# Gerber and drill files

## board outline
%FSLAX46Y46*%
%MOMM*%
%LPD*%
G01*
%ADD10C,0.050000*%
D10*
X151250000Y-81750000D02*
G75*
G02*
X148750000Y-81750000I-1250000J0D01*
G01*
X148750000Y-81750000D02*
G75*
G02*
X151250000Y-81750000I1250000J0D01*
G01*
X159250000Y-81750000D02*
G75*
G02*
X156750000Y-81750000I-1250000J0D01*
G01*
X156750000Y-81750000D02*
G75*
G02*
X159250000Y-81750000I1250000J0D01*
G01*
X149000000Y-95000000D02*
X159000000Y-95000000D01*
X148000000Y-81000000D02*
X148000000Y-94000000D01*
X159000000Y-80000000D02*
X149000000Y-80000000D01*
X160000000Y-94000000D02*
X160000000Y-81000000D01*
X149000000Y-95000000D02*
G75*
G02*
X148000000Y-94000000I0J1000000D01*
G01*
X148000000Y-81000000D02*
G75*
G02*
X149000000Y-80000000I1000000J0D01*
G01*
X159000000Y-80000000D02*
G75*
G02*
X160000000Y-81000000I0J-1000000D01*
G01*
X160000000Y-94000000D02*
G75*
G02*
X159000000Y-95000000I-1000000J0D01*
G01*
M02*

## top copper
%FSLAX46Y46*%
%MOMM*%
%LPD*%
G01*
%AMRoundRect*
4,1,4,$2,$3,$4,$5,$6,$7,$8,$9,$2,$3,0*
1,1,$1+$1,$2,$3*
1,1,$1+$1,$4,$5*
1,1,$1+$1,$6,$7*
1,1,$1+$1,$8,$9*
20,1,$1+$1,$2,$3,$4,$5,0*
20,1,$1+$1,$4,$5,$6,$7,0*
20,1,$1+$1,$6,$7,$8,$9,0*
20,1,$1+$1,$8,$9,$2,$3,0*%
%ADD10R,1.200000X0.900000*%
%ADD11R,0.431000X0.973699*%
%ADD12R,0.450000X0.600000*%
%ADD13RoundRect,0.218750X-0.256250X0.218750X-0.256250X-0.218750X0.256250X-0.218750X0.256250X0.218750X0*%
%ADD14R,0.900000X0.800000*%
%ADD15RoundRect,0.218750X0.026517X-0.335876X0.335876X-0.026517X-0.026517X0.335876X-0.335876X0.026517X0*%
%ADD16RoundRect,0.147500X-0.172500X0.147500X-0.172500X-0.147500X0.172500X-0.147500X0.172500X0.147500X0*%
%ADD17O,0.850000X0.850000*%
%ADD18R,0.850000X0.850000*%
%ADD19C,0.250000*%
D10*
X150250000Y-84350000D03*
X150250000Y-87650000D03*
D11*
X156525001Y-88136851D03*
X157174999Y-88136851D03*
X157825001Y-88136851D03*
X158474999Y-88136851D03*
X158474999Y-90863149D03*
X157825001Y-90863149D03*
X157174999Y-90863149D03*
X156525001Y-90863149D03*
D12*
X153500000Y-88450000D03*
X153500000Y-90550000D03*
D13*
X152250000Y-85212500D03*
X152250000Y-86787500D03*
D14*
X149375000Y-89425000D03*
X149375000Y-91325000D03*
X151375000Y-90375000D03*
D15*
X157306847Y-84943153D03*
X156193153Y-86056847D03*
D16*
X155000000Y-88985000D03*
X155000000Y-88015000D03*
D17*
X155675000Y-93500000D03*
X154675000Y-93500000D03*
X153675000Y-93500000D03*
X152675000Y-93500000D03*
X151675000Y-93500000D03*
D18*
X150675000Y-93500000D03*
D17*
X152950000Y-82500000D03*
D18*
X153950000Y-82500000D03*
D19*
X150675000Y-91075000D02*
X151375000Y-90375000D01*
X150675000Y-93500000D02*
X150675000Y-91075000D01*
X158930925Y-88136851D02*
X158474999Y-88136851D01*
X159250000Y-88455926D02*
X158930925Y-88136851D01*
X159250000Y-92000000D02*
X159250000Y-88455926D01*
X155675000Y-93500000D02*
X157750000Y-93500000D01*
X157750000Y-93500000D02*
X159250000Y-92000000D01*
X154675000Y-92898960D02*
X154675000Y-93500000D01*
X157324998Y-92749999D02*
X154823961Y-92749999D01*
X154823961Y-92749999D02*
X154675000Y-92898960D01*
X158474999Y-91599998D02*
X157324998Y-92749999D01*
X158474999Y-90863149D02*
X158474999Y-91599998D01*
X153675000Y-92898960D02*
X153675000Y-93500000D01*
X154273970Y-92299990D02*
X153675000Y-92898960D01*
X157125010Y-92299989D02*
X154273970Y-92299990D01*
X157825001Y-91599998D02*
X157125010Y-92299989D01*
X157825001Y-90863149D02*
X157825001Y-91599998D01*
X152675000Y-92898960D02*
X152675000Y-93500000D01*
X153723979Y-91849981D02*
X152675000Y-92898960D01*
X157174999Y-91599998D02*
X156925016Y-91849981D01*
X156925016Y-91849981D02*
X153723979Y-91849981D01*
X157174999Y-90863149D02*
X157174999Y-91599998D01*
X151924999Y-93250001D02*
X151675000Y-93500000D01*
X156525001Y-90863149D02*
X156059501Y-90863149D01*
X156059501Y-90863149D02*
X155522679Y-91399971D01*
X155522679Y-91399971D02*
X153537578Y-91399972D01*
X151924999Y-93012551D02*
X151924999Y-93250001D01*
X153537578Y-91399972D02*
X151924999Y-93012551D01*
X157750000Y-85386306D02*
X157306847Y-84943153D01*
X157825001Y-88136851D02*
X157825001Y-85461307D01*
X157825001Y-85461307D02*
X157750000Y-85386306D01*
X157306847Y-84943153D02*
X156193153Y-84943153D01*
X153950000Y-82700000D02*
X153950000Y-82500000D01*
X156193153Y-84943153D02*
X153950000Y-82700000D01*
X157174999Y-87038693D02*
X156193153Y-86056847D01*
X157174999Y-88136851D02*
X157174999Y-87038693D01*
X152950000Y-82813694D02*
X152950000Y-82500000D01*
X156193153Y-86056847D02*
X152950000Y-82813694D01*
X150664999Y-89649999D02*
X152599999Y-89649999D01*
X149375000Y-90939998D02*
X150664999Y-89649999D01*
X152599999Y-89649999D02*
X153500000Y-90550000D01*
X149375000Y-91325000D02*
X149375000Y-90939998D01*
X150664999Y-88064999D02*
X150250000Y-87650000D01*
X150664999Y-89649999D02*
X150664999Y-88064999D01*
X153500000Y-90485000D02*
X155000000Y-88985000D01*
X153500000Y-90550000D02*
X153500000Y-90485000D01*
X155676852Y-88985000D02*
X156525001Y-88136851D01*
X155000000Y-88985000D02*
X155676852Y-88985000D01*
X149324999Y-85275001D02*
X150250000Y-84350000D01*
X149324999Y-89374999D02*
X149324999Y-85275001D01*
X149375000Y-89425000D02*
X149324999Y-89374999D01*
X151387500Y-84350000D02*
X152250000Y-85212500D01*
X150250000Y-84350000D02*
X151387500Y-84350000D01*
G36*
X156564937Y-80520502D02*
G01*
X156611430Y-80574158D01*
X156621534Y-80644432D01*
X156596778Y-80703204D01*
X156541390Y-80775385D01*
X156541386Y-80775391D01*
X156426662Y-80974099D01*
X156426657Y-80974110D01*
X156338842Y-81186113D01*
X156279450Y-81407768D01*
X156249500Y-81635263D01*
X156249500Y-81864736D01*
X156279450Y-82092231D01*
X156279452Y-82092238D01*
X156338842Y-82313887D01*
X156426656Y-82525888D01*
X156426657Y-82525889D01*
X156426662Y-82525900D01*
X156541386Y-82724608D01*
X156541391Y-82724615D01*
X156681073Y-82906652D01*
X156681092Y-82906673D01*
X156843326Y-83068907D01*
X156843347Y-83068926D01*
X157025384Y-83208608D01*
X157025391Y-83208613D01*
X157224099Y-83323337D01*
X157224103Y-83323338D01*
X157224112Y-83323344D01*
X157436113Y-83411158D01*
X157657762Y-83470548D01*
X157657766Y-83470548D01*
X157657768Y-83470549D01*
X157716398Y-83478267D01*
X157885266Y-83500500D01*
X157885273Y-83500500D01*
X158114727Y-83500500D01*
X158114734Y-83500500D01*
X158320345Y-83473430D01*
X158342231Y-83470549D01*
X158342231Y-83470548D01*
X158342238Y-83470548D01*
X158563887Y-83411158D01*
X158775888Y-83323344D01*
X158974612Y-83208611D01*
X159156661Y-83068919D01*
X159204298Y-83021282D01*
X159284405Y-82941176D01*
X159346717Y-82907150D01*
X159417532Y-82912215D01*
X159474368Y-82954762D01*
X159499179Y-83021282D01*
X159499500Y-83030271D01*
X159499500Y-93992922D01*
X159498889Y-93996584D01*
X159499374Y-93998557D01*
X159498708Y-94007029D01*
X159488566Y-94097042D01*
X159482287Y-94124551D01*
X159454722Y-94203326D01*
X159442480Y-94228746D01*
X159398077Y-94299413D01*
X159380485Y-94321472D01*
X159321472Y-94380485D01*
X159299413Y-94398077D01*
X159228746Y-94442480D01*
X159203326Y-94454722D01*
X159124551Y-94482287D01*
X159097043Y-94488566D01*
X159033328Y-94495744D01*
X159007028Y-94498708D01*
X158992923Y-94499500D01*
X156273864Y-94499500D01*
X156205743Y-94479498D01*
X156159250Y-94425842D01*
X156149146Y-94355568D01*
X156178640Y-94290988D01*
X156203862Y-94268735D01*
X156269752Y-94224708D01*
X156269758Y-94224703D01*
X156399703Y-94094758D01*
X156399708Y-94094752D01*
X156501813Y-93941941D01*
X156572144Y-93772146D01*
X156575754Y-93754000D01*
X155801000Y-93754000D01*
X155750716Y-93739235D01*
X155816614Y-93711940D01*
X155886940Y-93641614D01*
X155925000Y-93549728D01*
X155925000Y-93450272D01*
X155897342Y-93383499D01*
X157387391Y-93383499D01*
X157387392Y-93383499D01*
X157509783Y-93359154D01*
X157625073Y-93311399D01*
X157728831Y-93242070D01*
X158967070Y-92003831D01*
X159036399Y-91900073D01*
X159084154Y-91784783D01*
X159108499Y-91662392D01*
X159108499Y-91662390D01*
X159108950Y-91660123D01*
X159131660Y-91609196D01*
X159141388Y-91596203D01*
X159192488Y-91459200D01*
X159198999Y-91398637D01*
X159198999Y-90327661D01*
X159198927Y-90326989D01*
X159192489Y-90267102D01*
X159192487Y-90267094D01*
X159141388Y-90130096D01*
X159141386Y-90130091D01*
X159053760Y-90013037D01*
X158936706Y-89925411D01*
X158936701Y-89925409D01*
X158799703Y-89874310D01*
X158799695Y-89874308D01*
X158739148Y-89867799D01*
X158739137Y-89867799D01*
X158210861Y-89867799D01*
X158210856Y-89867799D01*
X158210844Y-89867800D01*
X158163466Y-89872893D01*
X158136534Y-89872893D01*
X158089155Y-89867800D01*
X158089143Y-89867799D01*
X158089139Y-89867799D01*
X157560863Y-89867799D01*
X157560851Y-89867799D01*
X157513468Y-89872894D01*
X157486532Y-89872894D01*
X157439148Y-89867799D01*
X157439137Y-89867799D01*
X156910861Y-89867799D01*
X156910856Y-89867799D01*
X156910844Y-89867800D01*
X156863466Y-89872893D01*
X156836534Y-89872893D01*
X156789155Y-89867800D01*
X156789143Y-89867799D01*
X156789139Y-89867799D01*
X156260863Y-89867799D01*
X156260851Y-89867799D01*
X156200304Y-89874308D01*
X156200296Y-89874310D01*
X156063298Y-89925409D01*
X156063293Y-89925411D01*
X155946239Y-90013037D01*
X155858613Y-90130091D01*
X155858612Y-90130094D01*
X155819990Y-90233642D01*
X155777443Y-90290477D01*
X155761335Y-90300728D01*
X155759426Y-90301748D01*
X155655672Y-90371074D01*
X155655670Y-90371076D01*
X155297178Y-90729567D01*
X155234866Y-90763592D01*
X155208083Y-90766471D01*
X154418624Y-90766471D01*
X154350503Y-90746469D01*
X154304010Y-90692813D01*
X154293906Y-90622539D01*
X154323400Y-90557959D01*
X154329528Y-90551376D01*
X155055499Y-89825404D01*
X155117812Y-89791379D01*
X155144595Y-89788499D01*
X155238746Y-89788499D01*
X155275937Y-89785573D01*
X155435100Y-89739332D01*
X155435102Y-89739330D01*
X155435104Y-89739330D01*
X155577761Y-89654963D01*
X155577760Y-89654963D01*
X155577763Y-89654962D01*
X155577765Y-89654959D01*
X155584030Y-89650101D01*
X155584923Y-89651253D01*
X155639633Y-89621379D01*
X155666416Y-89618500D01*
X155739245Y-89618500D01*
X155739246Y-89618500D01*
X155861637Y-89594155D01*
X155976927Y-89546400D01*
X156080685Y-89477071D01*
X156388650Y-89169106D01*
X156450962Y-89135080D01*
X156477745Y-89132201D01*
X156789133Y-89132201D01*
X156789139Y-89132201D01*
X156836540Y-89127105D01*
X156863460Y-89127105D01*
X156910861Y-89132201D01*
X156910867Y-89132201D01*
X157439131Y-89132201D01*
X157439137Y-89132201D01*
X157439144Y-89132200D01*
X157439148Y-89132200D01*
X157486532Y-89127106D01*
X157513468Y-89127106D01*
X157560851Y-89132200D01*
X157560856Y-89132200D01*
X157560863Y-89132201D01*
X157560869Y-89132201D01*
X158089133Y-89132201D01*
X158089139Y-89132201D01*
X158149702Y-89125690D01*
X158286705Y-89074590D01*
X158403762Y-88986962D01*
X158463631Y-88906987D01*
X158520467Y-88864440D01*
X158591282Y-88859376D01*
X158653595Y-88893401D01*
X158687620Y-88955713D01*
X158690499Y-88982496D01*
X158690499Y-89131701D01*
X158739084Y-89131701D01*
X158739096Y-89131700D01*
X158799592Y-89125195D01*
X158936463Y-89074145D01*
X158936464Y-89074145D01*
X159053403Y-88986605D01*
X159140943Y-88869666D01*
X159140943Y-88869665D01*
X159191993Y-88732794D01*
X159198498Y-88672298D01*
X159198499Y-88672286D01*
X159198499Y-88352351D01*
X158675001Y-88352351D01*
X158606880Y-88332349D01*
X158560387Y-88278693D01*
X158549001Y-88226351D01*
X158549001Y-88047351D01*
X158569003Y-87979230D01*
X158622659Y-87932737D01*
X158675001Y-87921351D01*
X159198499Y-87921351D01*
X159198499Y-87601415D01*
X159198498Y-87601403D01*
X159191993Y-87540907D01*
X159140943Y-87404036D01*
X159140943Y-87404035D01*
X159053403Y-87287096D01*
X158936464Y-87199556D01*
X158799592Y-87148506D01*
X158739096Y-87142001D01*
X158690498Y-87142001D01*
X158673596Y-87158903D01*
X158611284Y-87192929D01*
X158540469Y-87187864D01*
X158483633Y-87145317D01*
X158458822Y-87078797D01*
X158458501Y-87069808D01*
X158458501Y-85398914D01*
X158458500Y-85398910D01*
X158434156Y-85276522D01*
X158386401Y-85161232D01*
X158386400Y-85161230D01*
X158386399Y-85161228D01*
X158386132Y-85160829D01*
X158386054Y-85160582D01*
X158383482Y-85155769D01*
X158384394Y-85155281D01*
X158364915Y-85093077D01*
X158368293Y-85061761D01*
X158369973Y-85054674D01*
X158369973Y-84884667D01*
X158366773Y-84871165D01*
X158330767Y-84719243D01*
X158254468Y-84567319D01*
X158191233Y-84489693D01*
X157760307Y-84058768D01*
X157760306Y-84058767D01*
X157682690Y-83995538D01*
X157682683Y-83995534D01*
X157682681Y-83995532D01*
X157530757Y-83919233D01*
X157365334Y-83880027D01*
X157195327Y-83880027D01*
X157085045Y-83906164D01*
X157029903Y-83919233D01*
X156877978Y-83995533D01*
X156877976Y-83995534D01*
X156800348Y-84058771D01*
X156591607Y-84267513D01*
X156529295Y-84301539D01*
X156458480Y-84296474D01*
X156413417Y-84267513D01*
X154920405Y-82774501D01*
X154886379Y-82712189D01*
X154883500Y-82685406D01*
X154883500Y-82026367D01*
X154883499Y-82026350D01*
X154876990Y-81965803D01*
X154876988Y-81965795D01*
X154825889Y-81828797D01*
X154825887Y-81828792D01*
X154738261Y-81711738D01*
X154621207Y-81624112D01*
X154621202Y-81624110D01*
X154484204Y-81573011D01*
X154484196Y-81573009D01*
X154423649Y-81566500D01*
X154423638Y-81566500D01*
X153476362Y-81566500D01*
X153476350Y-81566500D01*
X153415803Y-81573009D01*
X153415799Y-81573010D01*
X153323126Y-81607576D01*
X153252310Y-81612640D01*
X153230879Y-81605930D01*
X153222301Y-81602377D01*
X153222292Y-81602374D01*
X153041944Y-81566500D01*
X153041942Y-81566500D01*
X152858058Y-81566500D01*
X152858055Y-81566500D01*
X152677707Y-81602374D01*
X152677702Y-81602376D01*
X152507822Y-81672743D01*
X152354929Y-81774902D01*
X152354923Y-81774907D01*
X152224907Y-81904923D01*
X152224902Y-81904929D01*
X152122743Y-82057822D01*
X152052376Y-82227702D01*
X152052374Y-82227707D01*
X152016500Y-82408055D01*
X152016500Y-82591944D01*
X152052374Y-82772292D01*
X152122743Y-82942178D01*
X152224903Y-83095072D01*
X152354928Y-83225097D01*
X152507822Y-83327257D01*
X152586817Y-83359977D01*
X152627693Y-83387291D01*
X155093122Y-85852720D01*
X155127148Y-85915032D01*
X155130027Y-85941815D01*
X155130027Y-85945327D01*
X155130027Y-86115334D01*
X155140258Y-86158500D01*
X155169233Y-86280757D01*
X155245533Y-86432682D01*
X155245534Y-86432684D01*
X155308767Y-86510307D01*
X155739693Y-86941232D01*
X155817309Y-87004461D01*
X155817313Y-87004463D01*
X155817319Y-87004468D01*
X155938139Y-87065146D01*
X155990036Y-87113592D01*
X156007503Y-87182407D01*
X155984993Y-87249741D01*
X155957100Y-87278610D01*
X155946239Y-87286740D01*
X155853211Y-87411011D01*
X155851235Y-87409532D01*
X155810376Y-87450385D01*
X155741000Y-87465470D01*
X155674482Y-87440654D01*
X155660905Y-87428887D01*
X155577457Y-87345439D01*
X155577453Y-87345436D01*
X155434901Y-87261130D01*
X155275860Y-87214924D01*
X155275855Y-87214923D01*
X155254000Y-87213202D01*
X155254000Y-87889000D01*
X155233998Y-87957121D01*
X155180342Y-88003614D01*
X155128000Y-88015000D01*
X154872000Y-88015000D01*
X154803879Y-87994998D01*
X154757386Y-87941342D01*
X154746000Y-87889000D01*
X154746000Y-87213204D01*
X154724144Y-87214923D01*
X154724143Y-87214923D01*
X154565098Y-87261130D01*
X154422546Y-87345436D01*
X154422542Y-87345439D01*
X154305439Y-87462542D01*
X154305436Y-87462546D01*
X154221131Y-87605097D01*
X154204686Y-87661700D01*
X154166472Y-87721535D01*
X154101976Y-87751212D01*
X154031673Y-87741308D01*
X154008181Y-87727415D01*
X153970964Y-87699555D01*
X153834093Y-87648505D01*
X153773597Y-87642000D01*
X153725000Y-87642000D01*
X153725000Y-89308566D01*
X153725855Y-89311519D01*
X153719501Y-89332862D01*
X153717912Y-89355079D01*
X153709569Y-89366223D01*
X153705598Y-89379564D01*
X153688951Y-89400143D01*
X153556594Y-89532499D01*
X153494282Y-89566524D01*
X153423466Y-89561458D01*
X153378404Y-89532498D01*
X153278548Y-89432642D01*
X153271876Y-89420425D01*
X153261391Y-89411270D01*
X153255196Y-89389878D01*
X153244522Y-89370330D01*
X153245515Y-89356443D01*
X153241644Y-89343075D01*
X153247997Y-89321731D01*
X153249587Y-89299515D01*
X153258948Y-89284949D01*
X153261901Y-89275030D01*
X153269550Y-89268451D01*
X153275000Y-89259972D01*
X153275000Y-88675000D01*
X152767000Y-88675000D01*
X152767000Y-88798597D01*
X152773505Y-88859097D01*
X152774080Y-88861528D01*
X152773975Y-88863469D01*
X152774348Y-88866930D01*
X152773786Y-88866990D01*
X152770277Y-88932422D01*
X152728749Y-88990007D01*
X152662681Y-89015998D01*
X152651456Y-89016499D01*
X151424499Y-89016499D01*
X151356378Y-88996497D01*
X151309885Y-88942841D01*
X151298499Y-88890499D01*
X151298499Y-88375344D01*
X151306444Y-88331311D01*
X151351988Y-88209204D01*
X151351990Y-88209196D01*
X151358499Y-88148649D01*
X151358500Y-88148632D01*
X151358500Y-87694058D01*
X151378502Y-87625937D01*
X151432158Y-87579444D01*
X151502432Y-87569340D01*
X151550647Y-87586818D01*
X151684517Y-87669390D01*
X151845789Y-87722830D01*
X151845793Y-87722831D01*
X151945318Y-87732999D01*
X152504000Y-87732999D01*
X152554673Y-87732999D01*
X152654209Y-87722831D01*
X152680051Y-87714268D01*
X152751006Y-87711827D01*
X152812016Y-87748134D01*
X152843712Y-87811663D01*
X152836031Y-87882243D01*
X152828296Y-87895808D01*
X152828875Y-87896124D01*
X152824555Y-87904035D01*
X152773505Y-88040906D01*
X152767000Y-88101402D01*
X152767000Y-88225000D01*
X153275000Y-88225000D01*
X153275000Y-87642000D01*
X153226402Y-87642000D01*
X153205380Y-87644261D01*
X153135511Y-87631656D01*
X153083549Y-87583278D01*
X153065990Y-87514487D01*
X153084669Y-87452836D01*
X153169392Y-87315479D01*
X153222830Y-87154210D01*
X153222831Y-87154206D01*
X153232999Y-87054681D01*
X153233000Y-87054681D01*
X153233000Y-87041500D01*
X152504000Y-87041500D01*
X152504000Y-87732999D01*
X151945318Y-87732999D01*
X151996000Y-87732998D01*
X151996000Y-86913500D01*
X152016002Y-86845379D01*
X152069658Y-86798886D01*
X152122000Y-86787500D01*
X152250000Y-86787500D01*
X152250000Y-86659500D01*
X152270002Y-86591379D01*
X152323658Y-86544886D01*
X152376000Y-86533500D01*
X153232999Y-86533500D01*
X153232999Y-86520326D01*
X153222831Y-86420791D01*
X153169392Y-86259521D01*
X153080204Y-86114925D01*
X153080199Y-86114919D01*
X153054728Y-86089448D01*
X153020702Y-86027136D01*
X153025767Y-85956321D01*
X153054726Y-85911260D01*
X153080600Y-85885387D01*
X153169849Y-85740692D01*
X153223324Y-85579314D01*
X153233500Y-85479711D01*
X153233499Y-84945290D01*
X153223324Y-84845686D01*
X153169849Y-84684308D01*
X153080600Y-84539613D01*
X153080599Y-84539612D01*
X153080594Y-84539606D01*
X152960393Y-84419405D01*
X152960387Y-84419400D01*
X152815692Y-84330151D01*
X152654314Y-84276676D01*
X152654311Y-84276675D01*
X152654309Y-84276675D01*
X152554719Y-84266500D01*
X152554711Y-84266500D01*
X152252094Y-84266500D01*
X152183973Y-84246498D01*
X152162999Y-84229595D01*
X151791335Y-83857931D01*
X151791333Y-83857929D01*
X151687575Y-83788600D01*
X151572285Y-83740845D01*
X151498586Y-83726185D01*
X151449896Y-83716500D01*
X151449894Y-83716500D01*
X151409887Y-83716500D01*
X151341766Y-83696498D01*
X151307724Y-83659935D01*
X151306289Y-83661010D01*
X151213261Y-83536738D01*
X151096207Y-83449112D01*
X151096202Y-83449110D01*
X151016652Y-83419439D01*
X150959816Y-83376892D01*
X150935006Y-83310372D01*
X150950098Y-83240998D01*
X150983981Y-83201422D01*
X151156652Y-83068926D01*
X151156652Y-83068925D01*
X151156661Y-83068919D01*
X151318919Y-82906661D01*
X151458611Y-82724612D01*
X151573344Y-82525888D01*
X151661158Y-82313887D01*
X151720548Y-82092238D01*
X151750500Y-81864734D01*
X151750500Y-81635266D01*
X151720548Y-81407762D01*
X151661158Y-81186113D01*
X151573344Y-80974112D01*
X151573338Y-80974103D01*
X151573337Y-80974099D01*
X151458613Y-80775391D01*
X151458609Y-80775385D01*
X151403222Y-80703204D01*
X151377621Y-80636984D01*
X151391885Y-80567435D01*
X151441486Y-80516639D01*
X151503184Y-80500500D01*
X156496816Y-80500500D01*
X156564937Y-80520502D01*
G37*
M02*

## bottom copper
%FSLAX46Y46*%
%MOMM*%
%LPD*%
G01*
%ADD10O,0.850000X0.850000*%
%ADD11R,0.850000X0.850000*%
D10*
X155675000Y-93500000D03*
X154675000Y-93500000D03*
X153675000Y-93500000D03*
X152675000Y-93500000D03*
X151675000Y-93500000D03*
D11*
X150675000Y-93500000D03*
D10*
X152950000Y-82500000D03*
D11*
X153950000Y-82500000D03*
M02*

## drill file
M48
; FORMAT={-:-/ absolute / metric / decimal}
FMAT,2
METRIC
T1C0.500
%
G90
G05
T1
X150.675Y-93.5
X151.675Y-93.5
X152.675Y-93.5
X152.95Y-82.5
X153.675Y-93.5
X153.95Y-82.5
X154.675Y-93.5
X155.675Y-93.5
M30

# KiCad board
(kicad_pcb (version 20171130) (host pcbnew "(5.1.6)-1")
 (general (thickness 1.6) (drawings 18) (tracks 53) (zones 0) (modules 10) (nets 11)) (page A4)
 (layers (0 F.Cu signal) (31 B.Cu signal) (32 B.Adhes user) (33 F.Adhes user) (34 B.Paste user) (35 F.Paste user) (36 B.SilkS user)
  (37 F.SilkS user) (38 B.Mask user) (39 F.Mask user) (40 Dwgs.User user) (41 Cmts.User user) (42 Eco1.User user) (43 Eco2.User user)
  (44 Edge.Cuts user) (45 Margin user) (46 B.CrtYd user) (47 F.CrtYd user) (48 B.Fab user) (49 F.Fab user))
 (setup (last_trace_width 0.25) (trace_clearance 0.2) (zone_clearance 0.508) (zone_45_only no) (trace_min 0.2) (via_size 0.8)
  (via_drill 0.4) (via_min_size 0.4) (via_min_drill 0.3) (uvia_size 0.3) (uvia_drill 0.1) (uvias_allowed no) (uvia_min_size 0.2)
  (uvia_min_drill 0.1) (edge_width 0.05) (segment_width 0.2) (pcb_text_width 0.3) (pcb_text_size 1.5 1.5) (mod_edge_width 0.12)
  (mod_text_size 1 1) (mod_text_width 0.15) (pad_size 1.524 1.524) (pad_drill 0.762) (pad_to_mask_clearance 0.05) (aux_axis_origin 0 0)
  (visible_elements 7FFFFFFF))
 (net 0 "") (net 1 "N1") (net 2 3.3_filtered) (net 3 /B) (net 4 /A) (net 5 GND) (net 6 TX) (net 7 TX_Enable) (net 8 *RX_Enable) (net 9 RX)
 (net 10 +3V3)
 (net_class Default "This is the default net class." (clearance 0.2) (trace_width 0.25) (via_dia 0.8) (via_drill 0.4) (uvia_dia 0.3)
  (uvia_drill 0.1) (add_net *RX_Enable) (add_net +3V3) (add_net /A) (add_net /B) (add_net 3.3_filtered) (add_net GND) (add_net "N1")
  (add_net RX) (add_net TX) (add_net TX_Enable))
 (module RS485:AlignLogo (layer F.Cu) (at 158.25 93.25)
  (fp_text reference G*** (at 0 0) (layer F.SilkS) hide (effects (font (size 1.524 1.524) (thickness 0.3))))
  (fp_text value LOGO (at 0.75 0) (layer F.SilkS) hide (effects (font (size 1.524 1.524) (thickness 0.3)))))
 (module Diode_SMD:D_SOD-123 (layer F.Cu) (at 150.25 86 90)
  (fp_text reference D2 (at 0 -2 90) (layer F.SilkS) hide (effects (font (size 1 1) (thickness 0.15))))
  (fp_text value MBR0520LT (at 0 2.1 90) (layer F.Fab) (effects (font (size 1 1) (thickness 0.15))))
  (pad 2 smd rect (at 1.65 0 90) (size 0.9 1.2) (layers F.Cu F.Paste F.Mask) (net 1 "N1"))
  (pad 1 smd rect (at -1.65 0 90) (size 0.9 1.2) (layers F.Cu F.Paste F.Mask) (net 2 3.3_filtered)))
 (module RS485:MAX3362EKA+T (layer F.Cu) (at 157.5 89.5 90)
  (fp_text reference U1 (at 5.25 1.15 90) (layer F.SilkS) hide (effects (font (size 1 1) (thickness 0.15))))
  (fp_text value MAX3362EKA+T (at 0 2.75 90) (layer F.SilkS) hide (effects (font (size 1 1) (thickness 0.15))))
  (pad 8 smd rect (at 1.363149 -0.974999 90) (size 0.973699 0.431) (layers F.Cu F.Paste F.Mask) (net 2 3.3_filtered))
  (pad 7 smd rect (at 1.363149 -0.325001 90) (size 0.973699 0.431) (layers F.Cu F.Paste F.Mask) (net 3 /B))
  (pad 6 smd rect (at 1.363149 0.325001 90) (size 0.973699 0.431) (layers F.Cu F.Paste F.Mask) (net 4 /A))
  (pad 5 smd rect (at 1.363149 0.974999 90) (size 0.973699 0.431) (layers F.Cu F.Paste F.Mask) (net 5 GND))
  (pad 4 smd rect (at -1.363149 0.974999 90) (size 0.973699 0.431) (layers F.Cu F.Paste F.Mask) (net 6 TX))
  (pad 3 smd rect (at -1.363149 0.325001 90) (size 0.973699 0.431) (layers F.Cu F.Paste F.Mask) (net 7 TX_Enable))
  (pad 2 smd rect (at -1.363149 -0.325001 90) (size 0.973699 0.431) (layers F.Cu F.Paste F.Mask) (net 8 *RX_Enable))
  (pad 1 smd rect (at -1.363149 -0.974999 90) (size 0.973699 0.431) (layers F.Cu F.Paste F.Mask) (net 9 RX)))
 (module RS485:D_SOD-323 (layer F.Cu) (at 153.5 89.5 90)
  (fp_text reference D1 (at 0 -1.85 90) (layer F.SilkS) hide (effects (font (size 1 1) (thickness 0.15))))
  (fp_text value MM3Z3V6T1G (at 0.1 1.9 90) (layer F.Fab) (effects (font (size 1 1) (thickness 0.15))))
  (pad 2 smd rect (at 1.05 0 90) (size 0.6 0.45) (layers F.Cu F.Paste F.Mask) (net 5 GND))
  (pad 1 smd rect (at -1.05 0 90) (size 0.6 0.45) (layers F.Cu F.Paste F.Mask) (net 2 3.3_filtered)))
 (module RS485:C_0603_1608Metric (layer F.Cu) (at 152.25 86 270)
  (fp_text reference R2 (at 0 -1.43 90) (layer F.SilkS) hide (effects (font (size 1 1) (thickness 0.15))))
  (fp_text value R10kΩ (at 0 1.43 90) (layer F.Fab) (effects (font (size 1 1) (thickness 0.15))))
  (pad 1 smd roundrect (at -0.7875 0 270) (size 0.875 0.95) (layers F.Cu F.Paste F.Mask) (roundrect_rratio 0.25) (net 1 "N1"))
  (pad 2 smd roundrect (at 0.7875 0 270) (size 0.875 0.95) (layers F.Cu F.Paste F.Mask) (roundrect_rratio 0.25) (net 5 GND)))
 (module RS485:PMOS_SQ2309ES (layer F.Cu) (at 150.375 90.375)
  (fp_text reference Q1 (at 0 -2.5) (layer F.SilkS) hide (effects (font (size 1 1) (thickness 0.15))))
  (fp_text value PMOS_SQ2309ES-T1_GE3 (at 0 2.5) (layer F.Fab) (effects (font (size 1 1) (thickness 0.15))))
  (pad 1 smd rect (at -1 -0.95) (size 0.9 0.8) (layers F.Cu F.Paste F.Mask) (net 1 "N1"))
  (pad 2 smd rect (at -1 0.95) (size 0.9 0.8) (layers F.Cu F.Paste F.Mask) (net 2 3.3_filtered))
  (pad 3 smd rect (at 1 0) (size 0.9 0.8) (layers F.Cu F.Paste F.Mask) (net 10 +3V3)))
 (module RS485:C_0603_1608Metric (layer F.Cu) (at 156.75 85.5 45)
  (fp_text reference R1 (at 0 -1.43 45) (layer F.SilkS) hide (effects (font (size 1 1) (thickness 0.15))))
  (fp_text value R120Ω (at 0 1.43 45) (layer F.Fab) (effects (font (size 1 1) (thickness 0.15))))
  (pad 2 smd roundrect (at 0.7875 0 45) (size 0.875 0.95) (layers F.Cu F.Paste F.Mask) (roundrect_rratio 0.25) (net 4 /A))
  (pad 1 smd roundrect (at -0.7875 0 45) (size 0.875 0.95) (layers F.Cu F.Paste F.Mask) (roundrect_rratio 0.25) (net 3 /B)))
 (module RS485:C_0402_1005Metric (layer F.Cu) (at 155 88.5 270)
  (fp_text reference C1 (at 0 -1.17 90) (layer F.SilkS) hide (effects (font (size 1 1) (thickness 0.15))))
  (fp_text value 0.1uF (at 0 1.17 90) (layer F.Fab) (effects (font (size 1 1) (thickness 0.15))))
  (pad 2 smd roundrect (at 0.485 0 270) (size 0.59 0.64) (layers F.Cu F.Paste F.Mask) (roundrect_rratio 0.25) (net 2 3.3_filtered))
  (pad 1 smd roundrect (at -0.485 0 270) (size 0.59 0.64) (layers F.Cu F.Paste F.Mask) (roundrect_rratio 0.25) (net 5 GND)))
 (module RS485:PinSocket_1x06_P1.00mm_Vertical (layer F.Cu) (at 150.675 93.5 90)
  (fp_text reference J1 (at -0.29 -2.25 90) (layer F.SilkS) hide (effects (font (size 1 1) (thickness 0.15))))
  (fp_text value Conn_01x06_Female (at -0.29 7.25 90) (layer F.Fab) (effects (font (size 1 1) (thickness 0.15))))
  (pad 6 thru_hole oval (at 0 5 90) (size 0.85 0.85) (drill 0.5) (layers *.Cu *.Mask) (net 5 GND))
  (pad 5 thru_hole oval (at 0 4 90) (size 0.85 0.85) (drill 0.5) (layers *.Cu *.Mask) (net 6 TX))
  (pad 4 thru_hole oval (at 0 3 90) (size 0.85 0.85) (drill 0.5) (layers *.Cu *.Mask) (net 7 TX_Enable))
  (pad 3 thru_hole oval (at 0 2 90) (size 0.85 0.85) (drill 0.5) (layers *.Cu *.Mask) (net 8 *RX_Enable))
  (pad 2 thru_hole oval (at 0 1 90) (size 0.85 0.85) (drill 0.5) (layers *.Cu *.Mask) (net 9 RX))
  (pad 1 thru_hole rect (at 0 0 90) (size 0.85 0.85) (drill 0.5) (layers *.Cu *.Mask) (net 10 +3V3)))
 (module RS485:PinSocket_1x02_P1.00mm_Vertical (layer F.Cu) (at 153.95 82.5 270)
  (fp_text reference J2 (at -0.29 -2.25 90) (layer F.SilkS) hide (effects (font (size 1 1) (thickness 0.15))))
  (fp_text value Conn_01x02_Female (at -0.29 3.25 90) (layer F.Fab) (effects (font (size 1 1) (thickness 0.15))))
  (pad 2 thru_hole oval (at 0 1 270) (size 0.85 0.85) (drill 0.5) (layers *.Cu *.Mask) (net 3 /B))
  (pad 1 thru_hole rect (at 0 0 270) (size 0.85 0.85) (drill 0.5) (layers *.Cu *.Mask) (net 4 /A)))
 (gr_circle (center 150 81.75) (end 151 82.5) (layer Edge.Cuts) (width 0.05))
 (gr_circle (center 158 81.75) (end 158 83) (layer Edge.Cuts) (width 0.05))
 (gr_line (start 149 95) (end 159 95) (layer Edge.Cuts) (width 0.05))
 (gr_line (start 148 81) (end 148 94) (layer Edge.Cuts) (width 0.05))
 (gr_line (start 159 80) (end 149 80) (layer Edge.Cuts) (width 0.05))
 (gr_line (start 160 94) (end 160 81) (layer Edge.Cuts) (width 0.05))
 (gr_arc (start 149 94) (end 148 94) (angle -90) (layer Edge.Cuts) (width 0.05))
 (gr_arc (start 149 81) (end 149 80) (angle -90) (layer Edge.Cuts) (width 0.05))
 (gr_arc (start 159 81) (end 160 81) (angle -90) (layer Edge.Cuts) (width 0.05))
 (gr_arc (start 159 94) (end 159 95) (angle -90) (layer Edge.Cuts) (width 0.05))
 (segment (start 150.675 91.075) (end 151.375 90.375) (width 0.25) (layer F.Cu) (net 10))
 (segment (start 150.675 93.5) (end 150.675 91.075) (width 0.25) (layer F.Cu) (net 10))
 (segment (start 158.930925 88.136851) (end 158.474999 88.136851) (width 0.25) (layer F.Cu) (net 5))
 (segment (start 159.25 88.455926) (end 158.930925 88.136851) (width 0.25) (layer F.Cu) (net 5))
 (segment (start 159.25 92) (end 159.25 88.455926) (width 0.25) (layer F.Cu) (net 5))
 (segment (start 155.675 93.5) (end 157.75 93.5) (width 0.25) (layer F.Cu) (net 5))
 (segment (start 157.75 93.5) (end 159.25 92) (width 0.25) (layer F.Cu) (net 5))
 (segment (start 154.675 92.89896) (end 154.675 93.5) (width 0.25) (layer F.Cu) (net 6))
 (segment (start 157.324998 92.749999) (end 154.823961 92.749999) (width 0.25) (layer F.Cu) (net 6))
 (segment (start 154.823961 92.749999) (end 154.675 92.89896) (width 0.25) (layer F.Cu) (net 6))
 (segment (start 158.474999 91.599998) (end 157.324998 92.749999) (width 0.25) (layer F.Cu) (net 6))
 (segment (start 158.474999 90.863149) (end 158.474999 91.599998) (width 0.25) (layer F.Cu) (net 6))
 (segment (start 153.675 92.89896) (end 153.675 93.5) (width 0.25) (layer F.Cu) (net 7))
 (segment (start 154.27397 92.29999) (end 153.675 92.89896) (width 0.25) (layer F.Cu) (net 7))
 (segment (start 157.12501 92.299989) (end 154.27397 92.29999) (width 0.25) (layer F.Cu) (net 7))
 (segment (start 157.825001 91.599998) (end 157.12501 92.299989) (width 0.25) (layer F.Cu) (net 7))
 (segment (start 157.825001 90.863149) (end 157.825001 91.599998) (width 0.25) (layer F.Cu) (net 7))
 (segment (start 152.675 92.89896) (end 152.675 93.5) (width 0.25) (layer F.Cu) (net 8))
 (segment (start 153.723979 91.849981) (end 152.675 92.89896) (width 0.25) (layer F.Cu) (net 8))
 (segment (start 157.174999 91.599998) (end 156.925016 91.849981) (width 0.25) (layer F.Cu) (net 8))
 (segment (start 156.925016 91.849981) (end 153.723979 91.849981) (width 0.25) (layer F.Cu) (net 8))
 (segment (start 157.174999 90.863149) (end 157.174999 91.599998) (width 0.25) (layer F.Cu) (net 8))
 (segment (start 151.924999 93.250001) (end 151.675 93.5) (width 0.25) (layer F.Cu) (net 9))
 (segment (start 156.525001 90.863149) (end 156.059501 90.863149) (width 0.25) (layer F.Cu) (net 9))
 (segment (start 156.059501 90.863149) (end 155.522679 91.399971) (width 0.25) (layer F.Cu) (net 9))
 (segment (start 155.522679 91.399971) (end 153.537578 91.399972) (width 0.25) (layer F.Cu) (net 9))
 (segment (start 151.924999 93.012551) (end 151.924999 93.250001) (width 0.25) (layer F.Cu) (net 9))
 (segment (start 153.537578 91.399972) (end 151.924999 93.012551) (width 0.25) (layer F.Cu) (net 9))
 (segment (start 157.75 85.386306) (end 157.306847 84.943153) (width 0.25) (layer F.Cu) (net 4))
 (segment (start 157.825001 88.136851) (end 157.825001 85.461307) (width 0.25) (layer F.Cu) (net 4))
 (segment (start 157.825001 85.461307) (end 157.75 85.386306) (width 0.25) (layer F.Cu) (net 4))
 (segment (start 157.306847 84.943153) (end 156.193153 84.943153) (width 0.25) (layer F.Cu) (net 4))
 (segment (start 153.95 82.7) (end 153.95 82.5) (width 0.25) (layer F.Cu) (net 4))
 (segment (start 156.193153 84.943153) (end 153.95 82.7) (width 0.25) (layer F.Cu) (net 4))
 (segment (start 157.174999 87.038693) (end 156.193153 86.056847) (width 0.25) (layer F.Cu) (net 3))
 (segment (start 157.174999 88.136851) (end 157.174999 87.038693) (width 0.25) (layer F.Cu) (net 3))
 (segment (start 152.95 82.813694) (end 152.95 82.5) (width 0.25) (layer F.Cu) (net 3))
 (segment (start 156.193153 86.056847) (end 152.95 82.813694) (width 0.25) (layer F.Cu) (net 3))
 (segment (start 150.664999 89.649999) (end 152.599999 89.649999) (width 0.25) (layer F.Cu) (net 2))
 (segment (start 149.375 90.939998) (end 150.664999 89.649999) (width 0.25) (layer F.Cu) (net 2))
 (segment (start 152.599999 89.649999) (end 153.5 90.55) (width 0.25) (layer F.Cu) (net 2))
 (segment (start 149.375 91.325) (end 149.375 90.939998) (width 0.25) (layer F.Cu) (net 2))
 (segment (start 150.664999 88.064999) (end 150.25 87.65) (width 0.25) (layer F.Cu) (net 2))
 (segment (start 150.664999 89.649999) (end 150.664999 88.064999) (width 0.25) (layer F.Cu) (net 2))
 (segment (start 153.5 90.485) (end 155 88.985) (width 0.25) (layer F.Cu) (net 2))
 (segment (start 153.5 90.55) (end 153.5 90.485) (width 0.25) (layer F.Cu) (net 2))
 (segment (start 155.676852 88.985) (end 156.525001 88.136851) (width 0.25) (layer F.Cu) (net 2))
 (segment (start 155 88.985) (end 155.676852 88.985) (width 0.25) (layer F.Cu) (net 2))
 (segment (start 149.324999 85.275001) (end 150.25 84.35) (width 0.25) (layer F.Cu) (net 1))
 (segment (start 149.324999 89.374999) (end 149.324999 85.275001) (width 0.25) (layer F.Cu) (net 1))
 (segment (start 149.375 89.425) (end 149.324999 89.374999) (width 0.25) (layer F.Cu) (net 1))
 (segment (start 151.3875 84.35) (end 152.25 85.2125) (width 0.25) (layer F.Cu) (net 1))
 (segment (start 150.25 84.35) (end 151.3875 84.35) (width 0.25) (layer F.Cu) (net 1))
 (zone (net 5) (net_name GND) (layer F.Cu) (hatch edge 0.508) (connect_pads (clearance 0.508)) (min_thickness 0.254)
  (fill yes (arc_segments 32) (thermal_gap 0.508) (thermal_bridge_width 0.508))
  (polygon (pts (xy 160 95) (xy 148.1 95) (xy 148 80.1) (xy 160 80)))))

